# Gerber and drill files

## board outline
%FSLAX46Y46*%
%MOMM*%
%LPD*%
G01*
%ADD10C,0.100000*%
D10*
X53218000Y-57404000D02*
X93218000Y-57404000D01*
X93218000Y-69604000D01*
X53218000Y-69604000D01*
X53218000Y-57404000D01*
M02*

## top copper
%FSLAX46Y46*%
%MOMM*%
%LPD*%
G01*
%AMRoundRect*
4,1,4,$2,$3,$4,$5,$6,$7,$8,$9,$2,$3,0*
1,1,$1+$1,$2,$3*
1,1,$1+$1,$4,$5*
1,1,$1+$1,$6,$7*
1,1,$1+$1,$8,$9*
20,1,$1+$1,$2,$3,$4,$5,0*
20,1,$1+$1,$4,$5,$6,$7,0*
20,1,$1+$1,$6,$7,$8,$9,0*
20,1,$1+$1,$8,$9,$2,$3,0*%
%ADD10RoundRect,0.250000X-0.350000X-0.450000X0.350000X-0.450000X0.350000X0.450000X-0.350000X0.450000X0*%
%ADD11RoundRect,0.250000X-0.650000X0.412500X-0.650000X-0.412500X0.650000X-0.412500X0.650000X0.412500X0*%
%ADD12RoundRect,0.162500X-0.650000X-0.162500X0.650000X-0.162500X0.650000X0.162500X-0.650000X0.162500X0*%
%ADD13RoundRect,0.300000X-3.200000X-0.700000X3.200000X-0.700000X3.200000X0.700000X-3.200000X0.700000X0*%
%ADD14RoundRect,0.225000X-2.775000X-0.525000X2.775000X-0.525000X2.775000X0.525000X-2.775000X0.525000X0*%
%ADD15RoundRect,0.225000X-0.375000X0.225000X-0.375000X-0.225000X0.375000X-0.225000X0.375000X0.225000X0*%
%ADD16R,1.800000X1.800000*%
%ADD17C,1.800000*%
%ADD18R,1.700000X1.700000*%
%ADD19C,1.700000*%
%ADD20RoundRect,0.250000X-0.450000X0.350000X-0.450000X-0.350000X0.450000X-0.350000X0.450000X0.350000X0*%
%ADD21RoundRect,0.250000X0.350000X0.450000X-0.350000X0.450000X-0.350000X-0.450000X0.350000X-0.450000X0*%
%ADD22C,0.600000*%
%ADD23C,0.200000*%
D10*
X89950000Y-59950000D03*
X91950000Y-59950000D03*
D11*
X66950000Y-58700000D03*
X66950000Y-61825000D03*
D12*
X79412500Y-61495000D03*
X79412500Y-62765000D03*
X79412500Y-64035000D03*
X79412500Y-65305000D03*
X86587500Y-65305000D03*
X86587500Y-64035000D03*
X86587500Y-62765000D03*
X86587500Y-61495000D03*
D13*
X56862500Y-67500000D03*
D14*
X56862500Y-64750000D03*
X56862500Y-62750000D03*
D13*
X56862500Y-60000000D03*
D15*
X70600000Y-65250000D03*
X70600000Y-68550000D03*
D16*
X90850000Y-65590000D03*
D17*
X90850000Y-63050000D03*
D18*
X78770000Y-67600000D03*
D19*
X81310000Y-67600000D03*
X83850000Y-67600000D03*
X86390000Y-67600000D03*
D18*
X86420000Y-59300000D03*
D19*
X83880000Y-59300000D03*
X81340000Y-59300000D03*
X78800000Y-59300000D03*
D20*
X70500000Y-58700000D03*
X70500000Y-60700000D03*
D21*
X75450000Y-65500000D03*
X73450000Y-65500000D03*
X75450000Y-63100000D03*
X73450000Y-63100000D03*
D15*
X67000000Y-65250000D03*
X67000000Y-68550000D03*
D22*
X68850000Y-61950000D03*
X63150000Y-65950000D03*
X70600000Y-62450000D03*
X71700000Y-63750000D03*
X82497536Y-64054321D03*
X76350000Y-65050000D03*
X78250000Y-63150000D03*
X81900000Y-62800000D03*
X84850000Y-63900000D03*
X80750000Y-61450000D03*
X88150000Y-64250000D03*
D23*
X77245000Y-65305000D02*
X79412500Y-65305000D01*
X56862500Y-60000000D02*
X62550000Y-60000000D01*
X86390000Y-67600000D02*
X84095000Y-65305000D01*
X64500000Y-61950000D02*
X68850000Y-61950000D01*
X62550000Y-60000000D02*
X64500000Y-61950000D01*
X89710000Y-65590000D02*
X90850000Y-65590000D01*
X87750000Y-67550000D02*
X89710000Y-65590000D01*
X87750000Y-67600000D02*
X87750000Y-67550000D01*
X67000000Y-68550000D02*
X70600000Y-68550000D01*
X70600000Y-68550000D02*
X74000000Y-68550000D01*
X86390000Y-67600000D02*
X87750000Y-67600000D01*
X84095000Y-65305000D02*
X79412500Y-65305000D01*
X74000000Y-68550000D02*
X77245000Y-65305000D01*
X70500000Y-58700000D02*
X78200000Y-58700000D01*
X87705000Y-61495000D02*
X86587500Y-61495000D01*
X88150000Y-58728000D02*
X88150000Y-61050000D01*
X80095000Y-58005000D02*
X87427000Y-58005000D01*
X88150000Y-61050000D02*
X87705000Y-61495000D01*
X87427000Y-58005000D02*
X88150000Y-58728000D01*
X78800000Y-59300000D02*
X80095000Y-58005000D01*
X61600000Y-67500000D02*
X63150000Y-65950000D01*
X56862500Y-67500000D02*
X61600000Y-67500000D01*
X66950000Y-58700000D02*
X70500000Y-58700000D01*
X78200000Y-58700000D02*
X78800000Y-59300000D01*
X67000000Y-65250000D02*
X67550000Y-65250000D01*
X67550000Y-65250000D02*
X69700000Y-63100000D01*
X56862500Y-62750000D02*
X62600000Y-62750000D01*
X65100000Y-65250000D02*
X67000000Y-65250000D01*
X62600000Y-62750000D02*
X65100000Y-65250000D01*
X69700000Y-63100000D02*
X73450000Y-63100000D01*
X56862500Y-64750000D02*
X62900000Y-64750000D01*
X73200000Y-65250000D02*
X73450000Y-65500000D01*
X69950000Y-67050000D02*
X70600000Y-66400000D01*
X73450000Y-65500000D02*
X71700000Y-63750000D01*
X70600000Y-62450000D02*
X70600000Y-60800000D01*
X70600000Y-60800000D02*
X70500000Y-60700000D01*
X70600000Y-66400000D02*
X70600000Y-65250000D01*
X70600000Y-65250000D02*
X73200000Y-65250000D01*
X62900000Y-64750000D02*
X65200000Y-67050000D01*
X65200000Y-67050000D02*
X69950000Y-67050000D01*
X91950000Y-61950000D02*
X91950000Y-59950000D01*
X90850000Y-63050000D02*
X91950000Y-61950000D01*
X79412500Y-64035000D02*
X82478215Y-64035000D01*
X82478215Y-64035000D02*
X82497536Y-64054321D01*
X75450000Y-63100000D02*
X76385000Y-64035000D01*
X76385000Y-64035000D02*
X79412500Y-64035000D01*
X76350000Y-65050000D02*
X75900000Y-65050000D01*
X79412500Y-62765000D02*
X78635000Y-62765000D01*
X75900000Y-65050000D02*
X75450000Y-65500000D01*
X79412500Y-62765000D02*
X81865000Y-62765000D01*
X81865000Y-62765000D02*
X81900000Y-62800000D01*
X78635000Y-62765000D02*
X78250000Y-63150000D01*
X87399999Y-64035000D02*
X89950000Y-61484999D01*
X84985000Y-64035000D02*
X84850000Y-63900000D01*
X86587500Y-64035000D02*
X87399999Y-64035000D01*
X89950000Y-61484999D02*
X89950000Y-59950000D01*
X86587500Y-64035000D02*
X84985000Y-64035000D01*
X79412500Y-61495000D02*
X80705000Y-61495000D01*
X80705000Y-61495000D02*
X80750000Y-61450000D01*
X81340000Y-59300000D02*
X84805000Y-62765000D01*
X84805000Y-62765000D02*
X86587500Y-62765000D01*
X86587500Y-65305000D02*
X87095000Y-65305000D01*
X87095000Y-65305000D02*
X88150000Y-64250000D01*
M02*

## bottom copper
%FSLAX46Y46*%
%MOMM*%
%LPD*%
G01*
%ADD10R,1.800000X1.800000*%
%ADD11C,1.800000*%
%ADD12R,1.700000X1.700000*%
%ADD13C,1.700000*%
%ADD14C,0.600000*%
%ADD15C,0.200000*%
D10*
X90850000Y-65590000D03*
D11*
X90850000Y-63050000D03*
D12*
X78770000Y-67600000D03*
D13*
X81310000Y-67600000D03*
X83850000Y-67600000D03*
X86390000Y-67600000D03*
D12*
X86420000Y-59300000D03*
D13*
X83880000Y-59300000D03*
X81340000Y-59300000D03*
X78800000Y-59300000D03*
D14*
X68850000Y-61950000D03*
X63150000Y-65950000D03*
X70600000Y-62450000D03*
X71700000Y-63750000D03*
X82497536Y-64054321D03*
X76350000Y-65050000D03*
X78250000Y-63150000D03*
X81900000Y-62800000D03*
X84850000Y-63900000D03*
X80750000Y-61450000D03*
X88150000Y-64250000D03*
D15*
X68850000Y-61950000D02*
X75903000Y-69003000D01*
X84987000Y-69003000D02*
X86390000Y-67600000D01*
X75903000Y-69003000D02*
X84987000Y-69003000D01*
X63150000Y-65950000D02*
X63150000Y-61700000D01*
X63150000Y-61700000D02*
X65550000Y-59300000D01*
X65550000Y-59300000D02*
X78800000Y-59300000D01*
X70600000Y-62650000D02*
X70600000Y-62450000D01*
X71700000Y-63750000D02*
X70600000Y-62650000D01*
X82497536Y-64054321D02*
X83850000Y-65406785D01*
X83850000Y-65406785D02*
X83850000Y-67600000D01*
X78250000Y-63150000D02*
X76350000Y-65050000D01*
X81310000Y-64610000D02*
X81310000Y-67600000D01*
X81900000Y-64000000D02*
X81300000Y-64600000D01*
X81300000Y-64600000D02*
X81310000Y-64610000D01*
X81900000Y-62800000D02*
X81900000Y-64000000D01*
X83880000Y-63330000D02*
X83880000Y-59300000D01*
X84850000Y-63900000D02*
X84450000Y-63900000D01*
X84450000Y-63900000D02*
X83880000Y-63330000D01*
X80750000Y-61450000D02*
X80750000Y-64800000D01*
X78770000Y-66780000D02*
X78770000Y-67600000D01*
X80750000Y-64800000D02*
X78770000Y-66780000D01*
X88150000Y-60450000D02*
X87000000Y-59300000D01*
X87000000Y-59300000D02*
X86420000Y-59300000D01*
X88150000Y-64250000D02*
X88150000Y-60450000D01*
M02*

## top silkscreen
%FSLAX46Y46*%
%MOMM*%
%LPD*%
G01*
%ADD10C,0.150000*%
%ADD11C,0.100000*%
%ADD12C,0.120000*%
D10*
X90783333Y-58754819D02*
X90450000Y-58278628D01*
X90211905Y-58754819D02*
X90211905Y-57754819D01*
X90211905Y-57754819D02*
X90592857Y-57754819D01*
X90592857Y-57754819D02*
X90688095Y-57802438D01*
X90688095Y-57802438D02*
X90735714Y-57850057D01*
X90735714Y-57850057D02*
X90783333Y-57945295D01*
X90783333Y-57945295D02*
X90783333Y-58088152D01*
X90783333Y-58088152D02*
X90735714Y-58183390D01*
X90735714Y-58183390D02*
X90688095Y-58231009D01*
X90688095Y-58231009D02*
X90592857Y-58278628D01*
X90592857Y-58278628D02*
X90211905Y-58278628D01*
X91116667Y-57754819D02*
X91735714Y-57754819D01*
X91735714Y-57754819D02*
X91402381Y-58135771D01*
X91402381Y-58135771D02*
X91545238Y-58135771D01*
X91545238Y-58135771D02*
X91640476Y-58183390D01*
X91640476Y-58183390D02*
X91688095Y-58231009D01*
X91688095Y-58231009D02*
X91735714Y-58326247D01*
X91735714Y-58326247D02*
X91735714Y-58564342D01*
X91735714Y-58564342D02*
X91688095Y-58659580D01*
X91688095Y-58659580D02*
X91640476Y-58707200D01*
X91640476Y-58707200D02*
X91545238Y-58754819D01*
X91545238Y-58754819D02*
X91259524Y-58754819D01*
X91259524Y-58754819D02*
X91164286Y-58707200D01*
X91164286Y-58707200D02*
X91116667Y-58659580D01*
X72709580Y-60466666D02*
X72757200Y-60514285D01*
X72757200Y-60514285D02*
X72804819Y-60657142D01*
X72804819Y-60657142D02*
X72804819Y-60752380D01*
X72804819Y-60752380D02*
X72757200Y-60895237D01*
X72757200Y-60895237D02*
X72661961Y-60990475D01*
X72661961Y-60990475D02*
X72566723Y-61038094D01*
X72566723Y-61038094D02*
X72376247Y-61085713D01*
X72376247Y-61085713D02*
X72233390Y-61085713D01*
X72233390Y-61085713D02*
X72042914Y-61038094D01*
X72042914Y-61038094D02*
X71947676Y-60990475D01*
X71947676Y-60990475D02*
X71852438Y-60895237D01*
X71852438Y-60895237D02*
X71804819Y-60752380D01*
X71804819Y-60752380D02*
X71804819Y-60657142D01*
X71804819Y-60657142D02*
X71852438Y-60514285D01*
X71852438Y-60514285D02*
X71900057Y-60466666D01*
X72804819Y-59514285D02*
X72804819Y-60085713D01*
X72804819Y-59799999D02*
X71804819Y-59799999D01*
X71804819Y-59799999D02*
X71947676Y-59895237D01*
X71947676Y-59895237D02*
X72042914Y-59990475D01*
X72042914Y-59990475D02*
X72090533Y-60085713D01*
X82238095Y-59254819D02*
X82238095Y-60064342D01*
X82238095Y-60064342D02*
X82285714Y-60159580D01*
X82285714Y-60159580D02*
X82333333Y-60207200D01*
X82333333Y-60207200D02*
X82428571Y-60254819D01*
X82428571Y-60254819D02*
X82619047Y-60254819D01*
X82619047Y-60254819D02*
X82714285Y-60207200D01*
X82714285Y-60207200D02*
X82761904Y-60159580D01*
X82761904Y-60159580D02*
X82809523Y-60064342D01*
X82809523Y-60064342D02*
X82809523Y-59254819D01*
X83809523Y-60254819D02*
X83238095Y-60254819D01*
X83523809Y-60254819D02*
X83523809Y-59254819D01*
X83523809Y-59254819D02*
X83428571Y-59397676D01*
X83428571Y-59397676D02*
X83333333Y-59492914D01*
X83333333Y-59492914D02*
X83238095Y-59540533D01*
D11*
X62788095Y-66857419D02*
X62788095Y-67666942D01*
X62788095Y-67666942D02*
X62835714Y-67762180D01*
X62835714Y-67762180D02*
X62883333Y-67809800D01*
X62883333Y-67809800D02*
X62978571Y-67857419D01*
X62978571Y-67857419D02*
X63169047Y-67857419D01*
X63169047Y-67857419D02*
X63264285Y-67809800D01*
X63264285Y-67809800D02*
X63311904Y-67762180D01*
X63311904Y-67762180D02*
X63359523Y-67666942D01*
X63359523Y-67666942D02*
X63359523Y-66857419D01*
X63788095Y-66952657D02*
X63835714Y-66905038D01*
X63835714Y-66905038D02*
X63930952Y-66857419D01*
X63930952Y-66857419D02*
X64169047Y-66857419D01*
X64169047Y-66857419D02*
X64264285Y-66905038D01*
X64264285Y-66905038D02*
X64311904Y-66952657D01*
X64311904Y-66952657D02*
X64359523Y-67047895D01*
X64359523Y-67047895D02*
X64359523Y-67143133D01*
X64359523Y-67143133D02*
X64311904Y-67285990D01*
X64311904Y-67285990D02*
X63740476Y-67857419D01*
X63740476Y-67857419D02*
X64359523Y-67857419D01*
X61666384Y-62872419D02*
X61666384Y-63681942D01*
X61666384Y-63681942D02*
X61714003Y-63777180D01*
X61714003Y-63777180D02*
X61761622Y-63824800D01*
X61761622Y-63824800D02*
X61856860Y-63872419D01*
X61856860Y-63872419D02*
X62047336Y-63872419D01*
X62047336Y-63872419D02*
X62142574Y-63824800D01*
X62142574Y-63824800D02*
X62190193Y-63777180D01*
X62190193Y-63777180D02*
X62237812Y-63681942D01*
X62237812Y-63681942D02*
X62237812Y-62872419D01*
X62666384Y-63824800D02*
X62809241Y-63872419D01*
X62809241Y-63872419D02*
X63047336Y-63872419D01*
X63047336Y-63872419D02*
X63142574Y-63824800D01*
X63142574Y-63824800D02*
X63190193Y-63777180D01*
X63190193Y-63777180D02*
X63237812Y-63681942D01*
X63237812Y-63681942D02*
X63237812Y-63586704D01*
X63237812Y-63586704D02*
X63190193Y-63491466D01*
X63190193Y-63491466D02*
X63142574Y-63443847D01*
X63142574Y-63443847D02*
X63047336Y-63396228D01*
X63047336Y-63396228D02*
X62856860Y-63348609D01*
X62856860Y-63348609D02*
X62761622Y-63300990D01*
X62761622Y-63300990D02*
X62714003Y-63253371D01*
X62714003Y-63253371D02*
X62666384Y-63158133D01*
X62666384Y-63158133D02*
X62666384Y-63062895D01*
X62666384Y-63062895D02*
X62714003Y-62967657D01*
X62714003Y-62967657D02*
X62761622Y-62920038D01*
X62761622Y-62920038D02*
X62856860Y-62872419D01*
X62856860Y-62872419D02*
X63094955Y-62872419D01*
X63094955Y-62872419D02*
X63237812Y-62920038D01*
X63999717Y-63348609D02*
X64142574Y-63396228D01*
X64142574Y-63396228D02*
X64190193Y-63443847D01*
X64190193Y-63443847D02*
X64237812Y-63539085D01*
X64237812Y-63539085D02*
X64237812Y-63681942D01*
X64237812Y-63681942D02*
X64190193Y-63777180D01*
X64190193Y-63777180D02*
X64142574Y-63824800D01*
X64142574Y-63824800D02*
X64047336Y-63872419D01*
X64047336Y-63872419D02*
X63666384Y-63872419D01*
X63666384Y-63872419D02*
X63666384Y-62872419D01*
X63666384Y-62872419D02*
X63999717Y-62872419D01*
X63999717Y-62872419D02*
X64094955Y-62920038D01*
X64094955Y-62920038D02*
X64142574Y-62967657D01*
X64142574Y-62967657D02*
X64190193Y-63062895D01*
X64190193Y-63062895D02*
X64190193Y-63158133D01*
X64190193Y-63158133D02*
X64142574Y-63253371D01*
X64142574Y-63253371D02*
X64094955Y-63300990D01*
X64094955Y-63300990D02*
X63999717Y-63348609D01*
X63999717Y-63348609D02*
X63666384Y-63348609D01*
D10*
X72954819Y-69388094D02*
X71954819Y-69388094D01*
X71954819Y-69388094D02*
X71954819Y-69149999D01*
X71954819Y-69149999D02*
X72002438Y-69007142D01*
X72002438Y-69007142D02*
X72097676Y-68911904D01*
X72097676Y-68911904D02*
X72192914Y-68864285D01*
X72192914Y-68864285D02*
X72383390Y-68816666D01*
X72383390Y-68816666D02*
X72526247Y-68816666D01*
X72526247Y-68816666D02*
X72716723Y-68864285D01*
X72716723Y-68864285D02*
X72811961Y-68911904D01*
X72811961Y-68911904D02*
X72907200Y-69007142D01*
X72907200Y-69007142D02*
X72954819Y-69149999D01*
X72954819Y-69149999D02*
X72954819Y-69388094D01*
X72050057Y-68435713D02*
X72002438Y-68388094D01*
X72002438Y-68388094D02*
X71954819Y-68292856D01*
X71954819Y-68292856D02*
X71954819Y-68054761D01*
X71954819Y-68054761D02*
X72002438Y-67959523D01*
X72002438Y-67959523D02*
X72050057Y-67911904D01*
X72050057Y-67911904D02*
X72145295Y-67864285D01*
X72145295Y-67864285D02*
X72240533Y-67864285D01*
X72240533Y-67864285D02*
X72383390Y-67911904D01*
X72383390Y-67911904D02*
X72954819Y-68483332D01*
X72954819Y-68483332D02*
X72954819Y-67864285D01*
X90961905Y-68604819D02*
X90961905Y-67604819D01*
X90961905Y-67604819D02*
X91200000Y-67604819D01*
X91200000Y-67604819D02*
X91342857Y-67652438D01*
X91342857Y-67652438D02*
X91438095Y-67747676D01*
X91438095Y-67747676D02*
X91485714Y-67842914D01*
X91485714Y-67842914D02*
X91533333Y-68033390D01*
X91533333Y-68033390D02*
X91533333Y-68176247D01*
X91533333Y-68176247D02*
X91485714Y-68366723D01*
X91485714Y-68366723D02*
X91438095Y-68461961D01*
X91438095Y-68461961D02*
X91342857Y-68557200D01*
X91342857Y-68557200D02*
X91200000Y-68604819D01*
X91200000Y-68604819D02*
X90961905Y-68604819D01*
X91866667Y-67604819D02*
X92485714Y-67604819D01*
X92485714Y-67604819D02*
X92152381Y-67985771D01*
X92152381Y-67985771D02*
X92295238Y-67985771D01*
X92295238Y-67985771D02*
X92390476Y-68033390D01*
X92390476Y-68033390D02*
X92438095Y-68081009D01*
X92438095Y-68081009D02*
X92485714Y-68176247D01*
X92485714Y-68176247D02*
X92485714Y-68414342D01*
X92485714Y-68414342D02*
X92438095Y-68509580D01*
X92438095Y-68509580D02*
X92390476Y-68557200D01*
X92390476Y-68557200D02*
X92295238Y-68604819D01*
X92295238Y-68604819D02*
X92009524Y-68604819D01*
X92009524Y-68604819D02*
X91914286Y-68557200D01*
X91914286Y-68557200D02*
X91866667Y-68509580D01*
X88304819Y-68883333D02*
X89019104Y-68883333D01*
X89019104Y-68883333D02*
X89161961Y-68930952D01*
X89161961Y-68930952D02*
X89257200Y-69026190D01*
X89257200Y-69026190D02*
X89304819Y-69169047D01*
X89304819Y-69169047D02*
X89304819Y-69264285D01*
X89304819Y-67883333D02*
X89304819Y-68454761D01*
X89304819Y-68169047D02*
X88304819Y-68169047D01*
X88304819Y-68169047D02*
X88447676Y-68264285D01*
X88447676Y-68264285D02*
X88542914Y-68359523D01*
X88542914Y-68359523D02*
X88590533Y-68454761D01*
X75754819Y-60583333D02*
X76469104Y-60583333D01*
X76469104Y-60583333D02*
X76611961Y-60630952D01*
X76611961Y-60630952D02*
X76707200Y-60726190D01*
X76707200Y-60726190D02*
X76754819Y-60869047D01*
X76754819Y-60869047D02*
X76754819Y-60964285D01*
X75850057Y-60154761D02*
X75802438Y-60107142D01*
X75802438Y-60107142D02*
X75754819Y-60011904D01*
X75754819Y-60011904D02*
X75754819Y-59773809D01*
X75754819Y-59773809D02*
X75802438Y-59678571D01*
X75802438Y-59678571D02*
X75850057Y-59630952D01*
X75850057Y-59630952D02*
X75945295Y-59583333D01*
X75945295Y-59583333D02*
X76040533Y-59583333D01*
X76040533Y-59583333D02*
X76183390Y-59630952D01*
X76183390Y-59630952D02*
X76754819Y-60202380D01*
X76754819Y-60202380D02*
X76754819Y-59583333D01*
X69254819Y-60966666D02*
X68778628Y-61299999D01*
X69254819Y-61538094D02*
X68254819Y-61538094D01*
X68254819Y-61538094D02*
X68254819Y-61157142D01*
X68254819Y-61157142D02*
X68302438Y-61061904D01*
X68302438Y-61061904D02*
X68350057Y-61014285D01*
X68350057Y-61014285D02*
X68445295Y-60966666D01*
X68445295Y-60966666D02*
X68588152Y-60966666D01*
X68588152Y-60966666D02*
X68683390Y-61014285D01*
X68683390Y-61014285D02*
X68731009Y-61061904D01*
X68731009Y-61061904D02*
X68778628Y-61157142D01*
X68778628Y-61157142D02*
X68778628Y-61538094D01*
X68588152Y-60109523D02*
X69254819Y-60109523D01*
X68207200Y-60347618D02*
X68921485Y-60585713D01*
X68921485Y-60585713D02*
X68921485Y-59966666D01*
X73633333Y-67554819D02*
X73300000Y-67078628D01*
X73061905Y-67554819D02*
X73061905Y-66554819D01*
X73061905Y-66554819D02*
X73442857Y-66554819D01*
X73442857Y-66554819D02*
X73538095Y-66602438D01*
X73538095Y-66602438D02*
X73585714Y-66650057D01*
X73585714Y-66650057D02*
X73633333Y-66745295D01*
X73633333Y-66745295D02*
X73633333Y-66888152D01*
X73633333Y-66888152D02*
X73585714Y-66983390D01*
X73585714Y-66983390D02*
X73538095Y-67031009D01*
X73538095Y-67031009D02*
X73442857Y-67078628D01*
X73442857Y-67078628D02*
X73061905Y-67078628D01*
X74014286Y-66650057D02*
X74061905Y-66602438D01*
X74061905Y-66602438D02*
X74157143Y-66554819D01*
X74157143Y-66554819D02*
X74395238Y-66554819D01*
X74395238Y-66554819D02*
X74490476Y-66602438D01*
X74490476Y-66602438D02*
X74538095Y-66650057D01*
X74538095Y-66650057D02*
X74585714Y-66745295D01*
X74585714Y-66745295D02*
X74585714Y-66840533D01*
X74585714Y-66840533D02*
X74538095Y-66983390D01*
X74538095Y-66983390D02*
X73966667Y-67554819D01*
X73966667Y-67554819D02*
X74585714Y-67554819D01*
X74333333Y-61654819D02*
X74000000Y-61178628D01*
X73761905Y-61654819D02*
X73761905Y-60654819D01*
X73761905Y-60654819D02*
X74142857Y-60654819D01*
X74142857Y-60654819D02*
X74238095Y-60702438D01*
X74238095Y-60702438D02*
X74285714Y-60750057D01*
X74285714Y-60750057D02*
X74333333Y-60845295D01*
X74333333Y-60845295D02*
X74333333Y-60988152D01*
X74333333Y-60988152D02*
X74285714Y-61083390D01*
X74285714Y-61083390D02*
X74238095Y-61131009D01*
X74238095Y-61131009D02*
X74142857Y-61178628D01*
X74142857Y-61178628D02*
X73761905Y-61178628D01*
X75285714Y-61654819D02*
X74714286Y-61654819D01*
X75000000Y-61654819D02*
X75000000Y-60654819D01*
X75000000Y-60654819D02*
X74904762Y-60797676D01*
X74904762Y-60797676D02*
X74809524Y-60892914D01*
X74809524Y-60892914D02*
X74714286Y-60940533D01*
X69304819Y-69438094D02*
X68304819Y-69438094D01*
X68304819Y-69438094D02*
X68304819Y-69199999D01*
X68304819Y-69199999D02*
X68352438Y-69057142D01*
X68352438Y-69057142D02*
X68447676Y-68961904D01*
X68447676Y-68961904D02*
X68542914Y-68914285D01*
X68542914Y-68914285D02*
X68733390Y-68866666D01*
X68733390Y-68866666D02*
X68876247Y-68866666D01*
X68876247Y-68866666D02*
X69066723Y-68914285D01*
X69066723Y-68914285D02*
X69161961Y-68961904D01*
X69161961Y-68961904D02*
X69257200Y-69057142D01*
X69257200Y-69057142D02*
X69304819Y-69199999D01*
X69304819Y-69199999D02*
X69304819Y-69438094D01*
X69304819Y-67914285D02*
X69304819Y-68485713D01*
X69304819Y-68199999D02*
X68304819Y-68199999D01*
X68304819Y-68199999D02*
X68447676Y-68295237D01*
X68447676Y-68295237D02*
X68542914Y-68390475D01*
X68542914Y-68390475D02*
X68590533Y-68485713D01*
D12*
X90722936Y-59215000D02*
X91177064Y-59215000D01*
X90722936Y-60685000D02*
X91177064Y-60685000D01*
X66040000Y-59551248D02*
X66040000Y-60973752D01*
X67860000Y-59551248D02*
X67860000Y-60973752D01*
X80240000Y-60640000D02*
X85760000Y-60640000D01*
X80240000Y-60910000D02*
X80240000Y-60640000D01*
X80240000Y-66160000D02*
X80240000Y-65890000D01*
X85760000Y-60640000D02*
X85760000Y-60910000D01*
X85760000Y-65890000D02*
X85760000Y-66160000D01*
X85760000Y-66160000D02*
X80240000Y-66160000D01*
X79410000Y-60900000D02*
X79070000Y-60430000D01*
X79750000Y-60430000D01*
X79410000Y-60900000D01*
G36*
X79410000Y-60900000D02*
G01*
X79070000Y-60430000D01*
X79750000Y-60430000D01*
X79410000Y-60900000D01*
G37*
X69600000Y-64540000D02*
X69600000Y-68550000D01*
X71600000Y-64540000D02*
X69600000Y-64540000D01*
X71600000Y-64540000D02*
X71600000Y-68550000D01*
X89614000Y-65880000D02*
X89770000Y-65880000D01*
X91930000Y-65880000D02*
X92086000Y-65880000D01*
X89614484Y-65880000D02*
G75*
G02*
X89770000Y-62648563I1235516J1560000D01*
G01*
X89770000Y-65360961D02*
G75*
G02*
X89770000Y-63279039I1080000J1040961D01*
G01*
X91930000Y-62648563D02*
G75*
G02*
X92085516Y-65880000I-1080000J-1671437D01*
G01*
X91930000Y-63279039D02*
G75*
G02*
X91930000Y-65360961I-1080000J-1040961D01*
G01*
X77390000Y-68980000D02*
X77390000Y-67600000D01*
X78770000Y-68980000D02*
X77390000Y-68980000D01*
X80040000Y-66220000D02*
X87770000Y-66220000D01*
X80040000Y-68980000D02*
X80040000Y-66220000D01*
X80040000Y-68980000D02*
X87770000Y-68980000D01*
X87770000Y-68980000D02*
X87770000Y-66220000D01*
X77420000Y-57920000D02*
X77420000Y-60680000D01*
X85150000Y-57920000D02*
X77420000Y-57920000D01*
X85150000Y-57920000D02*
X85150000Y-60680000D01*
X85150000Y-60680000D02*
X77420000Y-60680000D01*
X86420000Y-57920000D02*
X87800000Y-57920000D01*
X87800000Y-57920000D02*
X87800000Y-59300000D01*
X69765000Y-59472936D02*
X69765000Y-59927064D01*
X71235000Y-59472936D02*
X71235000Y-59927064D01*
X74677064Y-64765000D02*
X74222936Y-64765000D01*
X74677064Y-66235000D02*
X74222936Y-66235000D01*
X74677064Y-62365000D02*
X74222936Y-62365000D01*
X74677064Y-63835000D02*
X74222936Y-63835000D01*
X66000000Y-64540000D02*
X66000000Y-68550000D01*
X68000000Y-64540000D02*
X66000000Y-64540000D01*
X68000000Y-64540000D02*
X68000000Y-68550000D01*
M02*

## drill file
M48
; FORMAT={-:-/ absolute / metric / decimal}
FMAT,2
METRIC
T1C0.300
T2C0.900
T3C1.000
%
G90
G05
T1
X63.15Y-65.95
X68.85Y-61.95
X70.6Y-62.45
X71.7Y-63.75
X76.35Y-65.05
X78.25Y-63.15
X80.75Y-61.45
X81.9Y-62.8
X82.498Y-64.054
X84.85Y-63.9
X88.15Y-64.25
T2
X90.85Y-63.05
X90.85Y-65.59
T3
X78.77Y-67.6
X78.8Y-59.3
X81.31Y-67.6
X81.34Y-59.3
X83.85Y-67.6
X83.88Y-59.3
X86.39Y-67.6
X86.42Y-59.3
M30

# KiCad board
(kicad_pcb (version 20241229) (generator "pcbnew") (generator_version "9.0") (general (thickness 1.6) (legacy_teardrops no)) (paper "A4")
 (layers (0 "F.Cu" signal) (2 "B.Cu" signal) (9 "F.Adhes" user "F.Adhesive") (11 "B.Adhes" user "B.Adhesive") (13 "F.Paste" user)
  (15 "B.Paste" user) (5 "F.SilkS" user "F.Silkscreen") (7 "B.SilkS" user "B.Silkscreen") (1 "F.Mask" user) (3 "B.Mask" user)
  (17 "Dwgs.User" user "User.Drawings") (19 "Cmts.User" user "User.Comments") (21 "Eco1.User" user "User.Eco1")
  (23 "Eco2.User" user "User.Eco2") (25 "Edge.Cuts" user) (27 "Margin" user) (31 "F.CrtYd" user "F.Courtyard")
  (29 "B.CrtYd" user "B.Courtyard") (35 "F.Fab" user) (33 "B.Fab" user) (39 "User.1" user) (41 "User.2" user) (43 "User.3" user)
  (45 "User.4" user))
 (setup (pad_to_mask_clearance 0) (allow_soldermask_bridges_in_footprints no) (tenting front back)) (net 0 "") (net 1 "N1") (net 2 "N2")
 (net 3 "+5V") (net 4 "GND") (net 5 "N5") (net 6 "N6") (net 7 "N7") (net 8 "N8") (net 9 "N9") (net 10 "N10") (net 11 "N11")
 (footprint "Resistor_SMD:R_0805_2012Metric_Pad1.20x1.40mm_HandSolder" (layer "F.Cu") (at 90.95 59.95)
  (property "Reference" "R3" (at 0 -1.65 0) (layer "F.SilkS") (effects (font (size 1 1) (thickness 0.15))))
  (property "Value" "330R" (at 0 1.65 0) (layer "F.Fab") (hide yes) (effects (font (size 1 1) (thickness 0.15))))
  (fp_line (start -0.227064 -0.735) (end 0.227064 -0.735) (stroke (width 0.12) (type solid)) (layer "F.SilkS"))
  (fp_line (start -0.227064 0.735) (end 0.227064 0.735) (stroke (width 0.12) (type solid)) (layer "F.SilkS"))
  (pad "1" smd roundrect (at -1 0) (size 1.2 1.4) (layers "F.Cu" "F.Mask" "F.Paste") (roundrect_rratio 0.208333) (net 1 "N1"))
  (pad "2" smd roundrect (at 1 0) (size 1.2 1.4) (layers "F.Cu" "F.Mask" "F.Paste") (roundrect_rratio 0.208333) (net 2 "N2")))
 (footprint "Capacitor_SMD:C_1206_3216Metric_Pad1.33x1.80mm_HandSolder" (layer "F.Cu") (at 66.95 60.2625 -90)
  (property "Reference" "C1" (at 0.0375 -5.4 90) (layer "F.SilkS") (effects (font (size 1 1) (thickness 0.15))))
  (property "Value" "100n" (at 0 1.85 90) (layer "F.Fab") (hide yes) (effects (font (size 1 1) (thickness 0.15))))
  (fp_line (start -0.711252 0.91) (end 0.711252 0.91) (stroke (width 0.12) (type solid)) (layer "F.SilkS"))
  (fp_line (start -0.711252 -0.91) (end 0.711252 -0.91) (stroke (width 0.12) (type solid)) (layer "F.SilkS"))
  (pad "1" smd roundrect (at -1.5625 0 270) (size 1.325 1.8) (layers "F.Cu" "F.Mask" "F.Paste") (roundrect_rratio 0.188679) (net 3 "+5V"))
  (pad "2" smd roundrect (at 1.5625 0 270) (size 1.325 1.8) (layers "F.Cu" "F.Mask" "F.Paste") (roundrect_rratio 0.188679) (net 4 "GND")))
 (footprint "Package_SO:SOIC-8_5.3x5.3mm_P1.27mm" (layer "F.Cu") (at 83 63.4)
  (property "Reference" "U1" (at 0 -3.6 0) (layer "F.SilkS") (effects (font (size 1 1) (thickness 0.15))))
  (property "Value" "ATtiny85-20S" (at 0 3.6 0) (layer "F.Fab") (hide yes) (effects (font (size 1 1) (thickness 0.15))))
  (fp_line (start -2.76 -2.76) (end 2.76 -2.76) (stroke (width 0.12) (type solid)) (layer "F.SilkS"))
  (fp_line (start -2.76 -2.49) (end -2.76 -2.76) (stroke (width 0.12) (type solid)) (layer "F.SilkS"))
  (fp_line (start -2.76 2.76) (end -2.76 2.49) (stroke (width 0.12) (type solid)) (layer "F.SilkS"))
  (fp_line (start 2.76 -2.76) (end 2.76 -2.49) (stroke (width 0.12) (type solid)) (layer "F.SilkS"))
  (fp_line (start 2.76 2.49) (end 2.76 2.76) (stroke (width 0.12) (type solid)) (layer "F.SilkS"))
  (fp_line (start 2.76 2.76) (end -2.76 2.76) (stroke (width 0.12) (type solid)) (layer "F.SilkS"))
  (fp_poly (pts (xy -3.59 -2.5) (xy -3.93 -2.97) (xy -3.25 -2.97)) (stroke (width 0.12) (type solid)) (fill yes) (layer "F.SilkS"))
  (pad "1" smd roundrect (at -3.5875 -1.905) (size 1.625 0.65) (layers "F.Cu" "F.Mask" "F.Paste") (roundrect_rratio 0.25) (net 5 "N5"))
  (pad "2" smd roundrect (at -3.5875 -0.635) (size 1.625 0.65) (layers "F.Cu" "F.Mask" "F.Paste") (roundrect_rratio 0.25) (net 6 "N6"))
  (pad "3" smd roundrect (at -3.5875 0.635) (size 1.625 0.65) (layers "F.Cu" "F.Mask" "F.Paste") (roundrect_rratio 0.25) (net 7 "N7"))
  (pad "4" smd roundrect (at -3.5875 1.905) (size 1.625 0.65) (layers "F.Cu" "F.Mask" "F.Paste") (roundrect_rratio 0.25) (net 4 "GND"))
  (pad "5" smd roundrect (at 3.5875 1.905) (size 1.625 0.65) (layers "F.Cu" "F.Mask" "F.Paste") (roundrect_rratio 0.25) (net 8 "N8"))
  (pad "6" smd roundrect (at 3.5875 0.635) (size 1.625 0.65) (layers "F.Cu" "F.Mask" "F.Paste") (roundrect_rratio 0.25) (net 1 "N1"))
  (pad "7" smd roundrect (at 3.5875 -0.635) (size 1.625 0.65) (layers "F.Cu" "F.Mask" "F.Paste") (roundrect_rratio 0.25) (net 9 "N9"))
  (pad "8" smd roundrect (at 3.5875 -1.905) (size 1.625 0.65) (layers "F.Cu" "F.Mask" "F.Paste") (roundrect_rratio 0.25) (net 3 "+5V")))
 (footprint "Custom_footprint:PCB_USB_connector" (layer "F.Cu") (at 56.8625 63.75)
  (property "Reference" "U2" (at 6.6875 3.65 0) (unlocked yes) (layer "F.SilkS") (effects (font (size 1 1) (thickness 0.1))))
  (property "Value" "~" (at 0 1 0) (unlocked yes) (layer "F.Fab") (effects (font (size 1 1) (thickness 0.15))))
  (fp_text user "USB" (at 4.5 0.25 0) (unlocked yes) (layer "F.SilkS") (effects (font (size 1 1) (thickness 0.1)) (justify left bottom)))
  (pad "1" smd roundrect (at 0 3.75) (size 7 2) (layers "F.Cu" "F.Mask" "F.Paste") (roundrect_rratio 0.15) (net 3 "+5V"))
  (pad "2" smd roundrect (at 0 1) (size 6 1.5) (layers "F.Cu" "F.Mask" "F.Paste") (roundrect_rratio 0.15) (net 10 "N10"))
  (pad "3" smd roundrect (at 0 -1) (size 6 1.5) (layers "F.Cu" "F.Mask" "F.Paste") (roundrect_rratio 0.15) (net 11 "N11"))
  (pad "4" smd roundrect (at 0 -3.75) (size 7 2) (layers "F.Cu" "F.Mask" "F.Paste") (roundrect_rratio 0.15) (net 4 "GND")))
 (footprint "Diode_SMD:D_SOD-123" (layer "F.Cu") (at 70.6 66.9 -90)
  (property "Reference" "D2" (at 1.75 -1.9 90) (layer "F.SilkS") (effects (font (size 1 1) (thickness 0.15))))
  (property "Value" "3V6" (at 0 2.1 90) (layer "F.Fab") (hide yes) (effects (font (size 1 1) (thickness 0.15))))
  (fp_line (start -2.36 1) (end 1.65 1) (stroke (width 0.12) (type solid)) (layer "F.SilkS"))
  (fp_line (start -2.36 -1) (end -2.36 1) (stroke (width 0.12) (type solid)) (layer "F.SilkS"))
  (fp_line (start -2.36 -1) (end 1.65 -1) (stroke (width 0.12) (type solid)) (layer "F.SilkS"))
  (pad "1" smd roundrect (at -1.65 0 270) (size 0.9 1.2) (layers "F.Cu" "F.Mask" "F.Paste") (roundrect_rratio 0.25) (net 10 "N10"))
  (pad "2" smd roundrect (at 1.65 0 270) (size 0.9 1.2) (layers "F.Cu" "F.Mask" "F.Paste") (roundrect_rratio 0.25) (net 4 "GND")))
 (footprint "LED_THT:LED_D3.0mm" (layer "F.Cu") (at 90.85 65.59 90)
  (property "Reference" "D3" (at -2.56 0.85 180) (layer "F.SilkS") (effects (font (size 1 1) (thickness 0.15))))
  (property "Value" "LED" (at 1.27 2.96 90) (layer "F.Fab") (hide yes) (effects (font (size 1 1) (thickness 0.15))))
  (fp_line (start -0.29 -1.236) (end -0.29 -1.08) (stroke (width 0.12) (type solid)) (layer "F.SilkS"))
  (fp_line (start -0.29 1.08) (end -0.29 1.236) (stroke (width 0.12) (type solid)) (layer "F.SilkS"))
  (fp_arc (start -0.29 -1.235516) (mid 1.36566 -1.987699) (end 2.941437 -1.08) (stroke (width 0.12) (type solid)) (layer "F.SilkS"))
  (fp_arc (start 0.229039 -1.08) (mid 1.27 -1.5) (end 2.310961 -1.08) (stroke (width 0.12) (type solid)) (layer "F.SilkS"))
  (fp_arc (start 2.941437 1.08) (mid 1.36566 1.987699) (end -0.29 1.235516) (stroke (width 0.12) (type solid)) (layer "F.SilkS"))
  (fp_arc (start 2.310961 1.08) (mid 1.27 1.5) (end 0.229039 1.08) (stroke (width 0.12) (type solid)) (layer "F.SilkS"))
  (pad "1" thru_hole rect (at 0 0 90) (size 1.8 1.8) (drill 0.9) (layers "*.Cu" "*.Mask") (remove_unused_layers no) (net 4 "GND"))
  (pad "2" thru_hole circle (at 2.54 0 90) (size 1.8 1.8) (drill 0.9) (layers "*.Cu" "*.Mask") (remove_unused_layers no) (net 2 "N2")))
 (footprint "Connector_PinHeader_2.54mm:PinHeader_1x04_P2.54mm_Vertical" (layer "F.Cu") (at 78.77 67.6 90)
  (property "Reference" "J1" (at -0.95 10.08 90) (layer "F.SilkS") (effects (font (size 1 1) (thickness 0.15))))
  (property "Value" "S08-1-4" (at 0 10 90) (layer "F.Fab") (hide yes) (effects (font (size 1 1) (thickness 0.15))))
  (fp_line (start -1.38 -1.38) (end 0 -1.38) (stroke (width 0.12) (type solid)) (layer "F.SilkS"))
  (fp_line (start -1.38 0) (end -1.38 -1.38) (stroke (width 0.12) (type solid)) (layer "F.SilkS"))
  (fp_line (start 1.38 1.27) (end 1.38 9) (stroke (width 0.12) (type solid)) (layer "F.SilkS"))
  (fp_line (start -1.38 1.27) (end 1.38 1.27) (stroke (width 0.12) (type solid)) (layer "F.SilkS"))
  (fp_line (start -1.38 1.27) (end -1.38 9) (stroke (width 0.12) (type solid)) (layer "F.SilkS"))
  (fp_line (start -1.38 9) (end 1.38 9) (stroke (width 0.12) (type solid)) (layer "F.SilkS"))
  (pad "1" thru_hole rect (at 0 0 90) (size 1.7 1.7) (drill 1) (layers "*.Cu" "*.Mask") (remove_unused_layers no) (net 5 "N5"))
  (pad "2" thru_hole circle (at 0 2.54 90) (size 1.7 1.7) (drill 1) (layers "*.Cu" "*.Mask") (remove_unused_layers no) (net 6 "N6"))
  (pad "3" thru_hole circle (at 0 5.08 90) (size 1.7 1.7) (drill 1) (layers "*.Cu" "*.Mask") (remove_unused_layers no) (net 7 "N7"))
  (pad "4" thru_hole circle (at 0 7.62 90) (size 1.7 1.7) (drill 1) (layers "*.Cu" "*.Mask") (remove_unused_layers no) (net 4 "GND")))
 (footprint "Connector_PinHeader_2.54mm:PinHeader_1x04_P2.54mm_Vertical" (layer "F.Cu") (at 86.42 59.3 -90)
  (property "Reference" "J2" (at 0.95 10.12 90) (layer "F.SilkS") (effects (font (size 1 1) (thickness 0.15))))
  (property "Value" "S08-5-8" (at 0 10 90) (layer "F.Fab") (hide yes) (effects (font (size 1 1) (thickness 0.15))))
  (fp_line (start -1.38 9) (end 1.38 9) (stroke (width 0.12) (type solid)) (layer "F.SilkS"))
  (fp_line (start -1.38 1.27) (end -1.38 9) (stroke (width 0.12) (type solid)) (layer "F.SilkS"))
  (fp_line (start -1.38 1.27) (end 1.38 1.27) (stroke (width 0.12) (type solid)) (layer "F.SilkS"))
  (fp_line (start 1.38 1.27) (end 1.38 9) (stroke (width 0.12) (type solid)) (layer "F.SilkS"))
  (fp_line (start -1.38 0) (end -1.38 -1.38) (stroke (width 0.12) (type solid)) (layer "F.SilkS"))
  (fp_line (start -1.38 -1.38) (end 0 -1.38) (stroke (width 0.12) (type solid)) (layer "F.SilkS"))
  (pad "1" thru_hole rect (at 0 0 270) (size 1.7 1.7) (drill 1) (layers "*.Cu" "*.Mask") (remove_unused_layers no) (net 8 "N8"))
  (pad "2" thru_hole circle (at 0 2.54 270) (size 1.7 1.7) (drill 1) (layers "*.Cu" "*.Mask") (remove_unused_layers no) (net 1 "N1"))
  (pad "3" thru_hole circle (at 0 5.08 270) (size 1.7 1.7) (drill 1) (layers "*.Cu" "*.Mask") (remove_unused_layers no) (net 9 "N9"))
  (pad "4" thru_hole circle (at 0 7.62 270) (size 1.7 1.7) (drill 1) (layers "*.Cu" "*.Mask") (remove_unused_layers no) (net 3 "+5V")))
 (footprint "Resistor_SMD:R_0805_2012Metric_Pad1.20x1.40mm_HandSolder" (layer "F.Cu") (at 70.5 59.7 -90)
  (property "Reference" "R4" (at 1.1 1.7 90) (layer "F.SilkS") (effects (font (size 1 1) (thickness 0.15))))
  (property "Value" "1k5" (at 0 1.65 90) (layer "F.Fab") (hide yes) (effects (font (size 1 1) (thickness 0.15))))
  (fp_line (start -0.227064 0.735) (end 0.227064 0.735) (stroke (width 0.12) (type solid)) (layer "F.SilkS"))
  (fp_line (start -0.227064 -0.735) (end 0.227064 -0.735) (stroke (width 0.12) (type solid)) (layer "F.SilkS"))
  (pad "1" smd roundrect (at -1 0 270) (size 1.2 1.4) (layers "F.Cu" "F.Mask" "F.Paste") (roundrect_rratio 0.208333) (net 3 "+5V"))
  (pad "2" smd roundrect (at 1 0 270) (size 1.2 1.4) (layers "F.Cu" "F.Mask" "F.Paste") (roundrect_rratio 0.208333) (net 10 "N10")))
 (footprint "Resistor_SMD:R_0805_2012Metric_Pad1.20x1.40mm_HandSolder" (layer "F.Cu") (at 74.45 65.5 180)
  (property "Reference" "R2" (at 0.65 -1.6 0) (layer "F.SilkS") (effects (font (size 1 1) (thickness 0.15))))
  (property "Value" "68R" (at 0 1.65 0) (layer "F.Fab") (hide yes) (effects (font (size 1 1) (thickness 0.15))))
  (fp_line (start -0.227064 0.735) (end 0.227064 0.735) (stroke (width 0.12) (type solid)) (layer "F.SilkS"))
  (fp_line (start -0.227064 -0.735) (end 0.227064 -0.735) (stroke (width 0.12) (type solid)) (layer "F.SilkS"))
  (pad "1" smd roundrect (at -1 0 180) (size 1.2 1.4) (layers "F.Cu" "F.Mask" "F.Paste") (roundrect_rratio 0.208333) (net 6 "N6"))
  (pad "2" smd roundrect (at 1 0 180) (size 1.2 1.4) (layers "F.Cu" "F.Mask" "F.Paste") (roundrect_rratio 0.208333) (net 10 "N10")))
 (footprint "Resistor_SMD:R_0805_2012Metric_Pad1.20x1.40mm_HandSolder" (layer "F.Cu") (at 74.45 63.1 180)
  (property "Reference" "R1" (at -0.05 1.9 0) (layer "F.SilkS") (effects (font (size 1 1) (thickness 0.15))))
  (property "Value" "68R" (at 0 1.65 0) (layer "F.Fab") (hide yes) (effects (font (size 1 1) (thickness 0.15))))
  (fp_line (start -0.227064 0.735) (end 0.227064 0.735) (stroke (width 0.12) (type solid)) (layer "F.SilkS"))
  (fp_line (start -0.227064 -0.735) (end 0.227064 -0.735) (stroke (width 0.12) (type solid)) (layer "F.SilkS"))
  (pad "1" smd roundrect (at -1 0 180) (size 1.2 1.4) (layers "F.Cu" "F.Mask" "F.Paste") (roundrect_rratio 0.208333) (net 7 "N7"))
  (pad "2" smd roundrect (at 1 0 180) (size 1.2 1.4) (layers "F.Cu" "F.Mask" "F.Paste") (roundrect_rratio 0.208333) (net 11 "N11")))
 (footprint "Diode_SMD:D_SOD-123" (layer "F.Cu") (at 67 66.9 -90)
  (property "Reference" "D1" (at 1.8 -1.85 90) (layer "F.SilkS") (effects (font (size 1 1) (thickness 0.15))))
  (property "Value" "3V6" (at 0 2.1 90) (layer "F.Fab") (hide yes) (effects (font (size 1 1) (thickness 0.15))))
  (fp_line (start -2.36 1) (end 1.65 1) (stroke (width 0.12) (type solid)) (layer "F.SilkS"))
  (fp_line (start -2.36 -1) (end -2.36 1) (stroke (width 0.12) (type solid)) (layer "F.SilkS"))
  (fp_line (start -2.36 -1) (end 1.65 -1) (stroke (width 0.12) (type solid)) (layer "F.SilkS"))
  (pad "1" smd roundrect (at -1.65 0 270) (size 0.9 1.2) (layers "F.Cu" "F.Mask" "F.Paste") (roundrect_rratio 0.25) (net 11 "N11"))
  (pad "2" smd roundrect (at 1.65 0 270) (size 0.9 1.2) (layers "F.Cu" "F.Mask" "F.Paste") (roundrect_rratio 0.25) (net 4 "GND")))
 (gr_rect (start 53.218 57.404) (end 93.218 69.604) (stroke (width 0.1) (type solid)) (fill no) (layer "Edge.Cuts"))
 (segment (start 77.245 65.305) (end 79.4125 65.305) (width 0.2) (layer "F.Cu") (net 4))
 (segment (start 56.8625 60) (end 62.55 60) (width 0.2) (layer "F.Cu") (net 4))
 (segment (start 86.39 67.6) (end 84.095 65.305) (width 0.2) (layer "F.Cu") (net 4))
 (segment (start 64.5 61.95) (end 68.85 61.95) (width 0.2) (layer "F.Cu") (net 4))
 (segment (start 62.55 60) (end 64.5 61.95) (width 0.2) (layer "F.Cu") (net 4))
 (segment (start 89.71 65.59) (end 90.85 65.59) (width 0.2) (layer "F.Cu") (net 4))
 (segment (start 87.75 67.55) (end 89.71 65.59) (width 0.2) (layer "F.Cu") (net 4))
 (segment (start 87.75 67.6) (end 87.75 67.55) (width 0.2) (layer "F.Cu") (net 4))
 (segment (start 67 68.55) (end 70.6 68.55) (width 0.2) (layer "F.Cu") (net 4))
 (segment (start 70.6 68.55) (end 74 68.55) (width 0.2) (layer "F.Cu") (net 4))
 (segment (start 86.39 67.6) (end 87.75 67.6) (width 0.2) (layer "F.Cu") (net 4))
 (segment (start 84.095 65.305) (end 79.4125 65.305) (width 0.2) (layer "F.Cu") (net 4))
 (segment (start 74 68.55) (end 77.245 65.305) (width 0.2) (layer "F.Cu") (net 4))
 (via (at 68.85 61.95) (size 0.6) (drill 0.3) (layers "F.Cu" "B.Cu") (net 4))
 (segment (start 68.85 61.95) (end 75.903 69.003) (width 0.2) (layer "B.Cu") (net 4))
 (segment (start 84.987 69.003) (end 86.39 67.6) (width 0.2) (layer "B.Cu") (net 4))
 (segment (start 75.903 69.003) (end 84.987 69.003) (width 0.2) (layer "B.Cu") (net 4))
 (segment (start 70.5 58.7) (end 78.2 58.7) (width 0.2) (layer "F.Cu") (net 3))
 (segment (start 87.705 61.495) (end 86.5875 61.495) (width 0.2) (layer "F.Cu") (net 3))
 (segment (start 88.15 58.728) (end 88.15 61.05) (width 0.2) (layer "F.Cu") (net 3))
 (segment (start 80.095 58.005) (end 87.427 58.005) (width 0.2) (layer "F.Cu") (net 3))
 (segment (start 88.15 61.05) (end 87.705 61.495) (width 0.2) (layer "F.Cu") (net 3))
 (segment (start 87.427 58.005) (end 88.15 58.728) (width 0.2) (layer "F.Cu") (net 3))
 (segment (start 78.8 59.3) (end 80.095 58.005) (width 0.2) (layer "F.Cu") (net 3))
 (segment (start 61.6 67.5) (end 63.15 65.95) (width 0.2) (layer "F.Cu") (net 3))
 (segment (start 56.8625 67.5) (end 61.6 67.5) (width 0.2) (layer "F.Cu") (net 3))
 (segment (start 66.95 58.7) (end 70.5 58.7) (width 0.2) (layer "F.Cu") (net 3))
 (segment (start 78.2 58.7) (end 78.8 59.3) (width 0.2) (layer "F.Cu") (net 3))
 (via (at 63.15 65.95) (size 0.6) (drill 0.3) (layers "F.Cu" "B.Cu") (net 3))
 (segment (start 63.15 65.95) (end 63.15 61.7) (width 0.2) (layer "B.Cu") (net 3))
 (segment (start 63.15 61.7) (end 65.55 59.3) (width 0.2) (layer "B.Cu") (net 3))
 (segment (start 65.55 59.3) (end 78.8 59.3) (width 0.2) (layer "B.Cu") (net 3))
 (segment (start 67 65.25) (end 67.55 65.25) (width 0.2) (layer "F.Cu") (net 11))
 (segment (start 67.55 65.25) (end 69.7 63.1) (width 0.2) (layer "F.Cu") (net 11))
 (segment (start 56.8625 62.75) (end 62.6 62.75) (width 0.2) (layer "F.Cu") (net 11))
 (segment (start 65.1 65.25) (end 67 65.25) (width 0.2) (layer "F.Cu") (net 11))
 (segment (start 62.6 62.75) (end 65.1 65.25) (width 0.2) (layer "F.Cu") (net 11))
 (segment (start 69.7 63.1) (end 73.45 63.1) (width 0.2) (layer "F.Cu") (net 11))
 (segment (start 56.8625 64.75) (end 62.9 64.75) (width 0.2) (layer "F.Cu") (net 10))
 (segment (start 73.2 65.25) (end 73.45 65.5) (width 0.2) (layer "F.Cu") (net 10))
 (segment (start 69.95 67.05) (end 70.6 66.4) (width 0.2) (layer "F.Cu") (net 10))
 (segment (start 73.45 65.5) (end 71.7 63.75) (width 0.2) (layer "F.Cu") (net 10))
 (segment (start 70.6 62.45) (end 70.6 60.8) (width 0.2) (layer "F.Cu") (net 10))
 (segment (start 70.6 60.8) (end 70.5 60.7) (width 0.2) (layer "F.Cu") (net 10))
 (segment (start 70.6 66.4) (end 70.6 65.25) (width 0.2) (layer "F.Cu") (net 10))
 (segment (start 70.6 65.25) (end 73.2 65.25) (width 0.2) (layer "F.Cu") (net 10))
 (segment (start 62.9 64.75) (end 65.2 67.05) (width 0.2) (layer "F.Cu") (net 10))
 (segment (start 65.2 67.05) (end 69.95 67.05) (width 0.2) (layer "F.Cu") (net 10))
 (via (at 70.6 62.45) (size 0.6) (drill 0.3) (layers "F.Cu" "B.Cu") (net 10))
 (via (at 71.7 63.75) (size 0.6) (drill 0.3) (layers "F.Cu" "B.Cu") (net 10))
 (segment (start 70.6 62.65) (end 70.6 62.45) (width 0.2) (layer "B.Cu") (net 10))
 (segment (start 71.7 63.75) (end 70.6 62.65) (width 0.2) (layer "B.Cu") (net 10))
 (segment (start 91.95 61.95) (end 91.95 59.95) (width 0.2) (layer "F.Cu") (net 2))
 (segment (start 90.85 63.05) (end 91.95 61.95) (width 0.2) (layer "F.Cu") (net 2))
 (segment (start 79.4125 64.035) (end 82.478215 64.035) (width 0.2) (layer "F.Cu") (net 7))
 (segment (start 82.478215 64.035) (end 82.497536 64.054321) (width 0.2) (layer "F.Cu") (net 7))
 (segment (start 75.45 63.1) (end 76.385 64.035) (width 0.2) (layer "F.Cu") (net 7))
 (segment (start 76.385 64.035) (end 79.4125 64.035) (width 0.2) (layer "F.Cu") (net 7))
 (via (at 82.497536 64.054321) (size 0.6) (drill 0.3) (layers "F.Cu" "B.Cu") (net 7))
 (segment (start 82.497536 64.054321) (end 83.85 65.406785) (width 0.2) (layer "B.Cu") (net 7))
 (segment (start 83.85 65.406785) (end 83.85 67.6) (width 0.2) (layer "B.Cu") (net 7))
 (segment (start 76.35 65.05) (end 75.9 65.05) (width 0.2) (layer "F.Cu") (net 6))
 (segment (start 79.4125 62.765) (end 78.635 62.765) (width 0.2) (layer "F.Cu") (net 6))
 (segment (start 75.9 65.05) (end 75.45 65.5) (width 0.2) (layer "F.Cu") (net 6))
 (segment (start 79.4125 62.765) (end 81.865 62.765) (width 0.2) (layer "F.Cu") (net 6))
 (segment (start 81.865 62.765) (end 81.9 62.8) (width 0.2) (layer "F.Cu") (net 6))
 (segment (start 78.635 62.765) (end 78.25 63.15) (width 0.2) (layer "F.Cu") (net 6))
 (via (at 76.35 65.05) (size 0.6) (drill 0.3) (layers "F.Cu" "B.Cu") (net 6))
 (via (at 78.25 63.15) (size 0.6) (drill 0.3) (layers "F.Cu" "B.Cu") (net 6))
 (via (at 81.9 62.8) (size 0.6) (drill 0.3) (layers "F.Cu" "B.Cu") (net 6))
 (segment (start 78.25 63.15) (end 76.35 65.05) (width 0.2) (layer "B.Cu") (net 6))
 (segment (start 81.31 64.61) (end 81.31 67.6) (width 0.2) (layer "B.Cu") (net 6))
 (segment (start 81.9 64) (end 81.3 64.6) (width 0.2) (layer "B.Cu") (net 6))
 (segment (start 81.3 64.6) (end 81.31 64.61) (width 0.2) (layer "B.Cu") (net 6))
 (segment (start 81.9 62.8) (end 81.9 64) (width 0.2) (layer "B.Cu") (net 6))
 (segment (start 87.399999 64.035) (end 89.95 61.484999) (width 0.2) (layer "F.Cu") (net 1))
 (segment (start 84.985 64.035) (end 84.85 63.9) (width 0.2) (layer "F.Cu") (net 1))
 (segment (start 86.5875 64.035) (end 87.399999 64.035) (width 0.2) (layer "F.Cu") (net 1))
 (segment (start 89.95 61.484999) (end 89.95 59.95) (width 0.2) (layer "F.Cu") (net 1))
 (segment (start 86.5875 64.035) (end 84.985 64.035) (width 0.2) (layer "F.Cu") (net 1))
 (via (at 84.85 63.9) (size 0.6) (drill 0.3) (layers "F.Cu" "B.Cu") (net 1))
 (segment (start 83.88 63.33) (end 83.88 59.3) (width 0.2) (layer "B.Cu") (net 1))
 (segment (start 84.85 63.9) (end 84.45 63.9) (width 0.2) (layer "B.Cu") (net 1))
 (segment (start 84.45 63.9) (end 83.88 63.33) (width 0.2) (layer "B.Cu") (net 1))
 (segment (start 79.4125 61.495) (end 80.705 61.495) (width 0.2) (layer "F.Cu") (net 5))
 (segment (start 80.705 61.495) (end 80.75 61.45) (width 0.2) (layer "F.Cu") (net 5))
 (via (at 80.75 61.45) (size 0.6) (drill 0.3) (layers "F.Cu" "B.Cu") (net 5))
 (segment (start 80.75 61.45) (end 80.75 64.8) (width 0.2) (layer "B.Cu") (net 5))
 (segment (start 78.77 66.78) (end 78.77 67.6) (width 0.2) (layer "B.Cu") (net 5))
 (segment (start 80.75 64.8) (end 78.77 66.78) (width 0.2) (layer "B.Cu") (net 5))
 (segment (start 81.34 59.3) (end 84.805 62.765) (width 0.2) (layer "F.Cu") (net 9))
 (segment (start 84.805 62.765) (end 86.5875 62.765) (width 0.2) (layer "F.Cu") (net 9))
 (segment (start 86.5875 65.305) (end 87.095 65.305) (width 0.2) (layer "F.Cu") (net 8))
 (segment (start 87.095 65.305) (end 88.15 64.25) (width 0.2) (layer "F.Cu") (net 8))
 (via (at 88.15 64.25) (size 0.6) (drill 0.3) (layers "F.Cu" "B.Cu") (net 8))
 (segment (start 88.15 60.45) (end 87 59.3) (width 0.2) (layer "B.Cu") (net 8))
 (segment (start 87 59.3) (end 86.42 59.3) (width 0.2) (layer "B.Cu") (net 8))
 (segment (start 88.15 64.25) (end 88.15 60.45) (width 0.2) (layer "B.Cu") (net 8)))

